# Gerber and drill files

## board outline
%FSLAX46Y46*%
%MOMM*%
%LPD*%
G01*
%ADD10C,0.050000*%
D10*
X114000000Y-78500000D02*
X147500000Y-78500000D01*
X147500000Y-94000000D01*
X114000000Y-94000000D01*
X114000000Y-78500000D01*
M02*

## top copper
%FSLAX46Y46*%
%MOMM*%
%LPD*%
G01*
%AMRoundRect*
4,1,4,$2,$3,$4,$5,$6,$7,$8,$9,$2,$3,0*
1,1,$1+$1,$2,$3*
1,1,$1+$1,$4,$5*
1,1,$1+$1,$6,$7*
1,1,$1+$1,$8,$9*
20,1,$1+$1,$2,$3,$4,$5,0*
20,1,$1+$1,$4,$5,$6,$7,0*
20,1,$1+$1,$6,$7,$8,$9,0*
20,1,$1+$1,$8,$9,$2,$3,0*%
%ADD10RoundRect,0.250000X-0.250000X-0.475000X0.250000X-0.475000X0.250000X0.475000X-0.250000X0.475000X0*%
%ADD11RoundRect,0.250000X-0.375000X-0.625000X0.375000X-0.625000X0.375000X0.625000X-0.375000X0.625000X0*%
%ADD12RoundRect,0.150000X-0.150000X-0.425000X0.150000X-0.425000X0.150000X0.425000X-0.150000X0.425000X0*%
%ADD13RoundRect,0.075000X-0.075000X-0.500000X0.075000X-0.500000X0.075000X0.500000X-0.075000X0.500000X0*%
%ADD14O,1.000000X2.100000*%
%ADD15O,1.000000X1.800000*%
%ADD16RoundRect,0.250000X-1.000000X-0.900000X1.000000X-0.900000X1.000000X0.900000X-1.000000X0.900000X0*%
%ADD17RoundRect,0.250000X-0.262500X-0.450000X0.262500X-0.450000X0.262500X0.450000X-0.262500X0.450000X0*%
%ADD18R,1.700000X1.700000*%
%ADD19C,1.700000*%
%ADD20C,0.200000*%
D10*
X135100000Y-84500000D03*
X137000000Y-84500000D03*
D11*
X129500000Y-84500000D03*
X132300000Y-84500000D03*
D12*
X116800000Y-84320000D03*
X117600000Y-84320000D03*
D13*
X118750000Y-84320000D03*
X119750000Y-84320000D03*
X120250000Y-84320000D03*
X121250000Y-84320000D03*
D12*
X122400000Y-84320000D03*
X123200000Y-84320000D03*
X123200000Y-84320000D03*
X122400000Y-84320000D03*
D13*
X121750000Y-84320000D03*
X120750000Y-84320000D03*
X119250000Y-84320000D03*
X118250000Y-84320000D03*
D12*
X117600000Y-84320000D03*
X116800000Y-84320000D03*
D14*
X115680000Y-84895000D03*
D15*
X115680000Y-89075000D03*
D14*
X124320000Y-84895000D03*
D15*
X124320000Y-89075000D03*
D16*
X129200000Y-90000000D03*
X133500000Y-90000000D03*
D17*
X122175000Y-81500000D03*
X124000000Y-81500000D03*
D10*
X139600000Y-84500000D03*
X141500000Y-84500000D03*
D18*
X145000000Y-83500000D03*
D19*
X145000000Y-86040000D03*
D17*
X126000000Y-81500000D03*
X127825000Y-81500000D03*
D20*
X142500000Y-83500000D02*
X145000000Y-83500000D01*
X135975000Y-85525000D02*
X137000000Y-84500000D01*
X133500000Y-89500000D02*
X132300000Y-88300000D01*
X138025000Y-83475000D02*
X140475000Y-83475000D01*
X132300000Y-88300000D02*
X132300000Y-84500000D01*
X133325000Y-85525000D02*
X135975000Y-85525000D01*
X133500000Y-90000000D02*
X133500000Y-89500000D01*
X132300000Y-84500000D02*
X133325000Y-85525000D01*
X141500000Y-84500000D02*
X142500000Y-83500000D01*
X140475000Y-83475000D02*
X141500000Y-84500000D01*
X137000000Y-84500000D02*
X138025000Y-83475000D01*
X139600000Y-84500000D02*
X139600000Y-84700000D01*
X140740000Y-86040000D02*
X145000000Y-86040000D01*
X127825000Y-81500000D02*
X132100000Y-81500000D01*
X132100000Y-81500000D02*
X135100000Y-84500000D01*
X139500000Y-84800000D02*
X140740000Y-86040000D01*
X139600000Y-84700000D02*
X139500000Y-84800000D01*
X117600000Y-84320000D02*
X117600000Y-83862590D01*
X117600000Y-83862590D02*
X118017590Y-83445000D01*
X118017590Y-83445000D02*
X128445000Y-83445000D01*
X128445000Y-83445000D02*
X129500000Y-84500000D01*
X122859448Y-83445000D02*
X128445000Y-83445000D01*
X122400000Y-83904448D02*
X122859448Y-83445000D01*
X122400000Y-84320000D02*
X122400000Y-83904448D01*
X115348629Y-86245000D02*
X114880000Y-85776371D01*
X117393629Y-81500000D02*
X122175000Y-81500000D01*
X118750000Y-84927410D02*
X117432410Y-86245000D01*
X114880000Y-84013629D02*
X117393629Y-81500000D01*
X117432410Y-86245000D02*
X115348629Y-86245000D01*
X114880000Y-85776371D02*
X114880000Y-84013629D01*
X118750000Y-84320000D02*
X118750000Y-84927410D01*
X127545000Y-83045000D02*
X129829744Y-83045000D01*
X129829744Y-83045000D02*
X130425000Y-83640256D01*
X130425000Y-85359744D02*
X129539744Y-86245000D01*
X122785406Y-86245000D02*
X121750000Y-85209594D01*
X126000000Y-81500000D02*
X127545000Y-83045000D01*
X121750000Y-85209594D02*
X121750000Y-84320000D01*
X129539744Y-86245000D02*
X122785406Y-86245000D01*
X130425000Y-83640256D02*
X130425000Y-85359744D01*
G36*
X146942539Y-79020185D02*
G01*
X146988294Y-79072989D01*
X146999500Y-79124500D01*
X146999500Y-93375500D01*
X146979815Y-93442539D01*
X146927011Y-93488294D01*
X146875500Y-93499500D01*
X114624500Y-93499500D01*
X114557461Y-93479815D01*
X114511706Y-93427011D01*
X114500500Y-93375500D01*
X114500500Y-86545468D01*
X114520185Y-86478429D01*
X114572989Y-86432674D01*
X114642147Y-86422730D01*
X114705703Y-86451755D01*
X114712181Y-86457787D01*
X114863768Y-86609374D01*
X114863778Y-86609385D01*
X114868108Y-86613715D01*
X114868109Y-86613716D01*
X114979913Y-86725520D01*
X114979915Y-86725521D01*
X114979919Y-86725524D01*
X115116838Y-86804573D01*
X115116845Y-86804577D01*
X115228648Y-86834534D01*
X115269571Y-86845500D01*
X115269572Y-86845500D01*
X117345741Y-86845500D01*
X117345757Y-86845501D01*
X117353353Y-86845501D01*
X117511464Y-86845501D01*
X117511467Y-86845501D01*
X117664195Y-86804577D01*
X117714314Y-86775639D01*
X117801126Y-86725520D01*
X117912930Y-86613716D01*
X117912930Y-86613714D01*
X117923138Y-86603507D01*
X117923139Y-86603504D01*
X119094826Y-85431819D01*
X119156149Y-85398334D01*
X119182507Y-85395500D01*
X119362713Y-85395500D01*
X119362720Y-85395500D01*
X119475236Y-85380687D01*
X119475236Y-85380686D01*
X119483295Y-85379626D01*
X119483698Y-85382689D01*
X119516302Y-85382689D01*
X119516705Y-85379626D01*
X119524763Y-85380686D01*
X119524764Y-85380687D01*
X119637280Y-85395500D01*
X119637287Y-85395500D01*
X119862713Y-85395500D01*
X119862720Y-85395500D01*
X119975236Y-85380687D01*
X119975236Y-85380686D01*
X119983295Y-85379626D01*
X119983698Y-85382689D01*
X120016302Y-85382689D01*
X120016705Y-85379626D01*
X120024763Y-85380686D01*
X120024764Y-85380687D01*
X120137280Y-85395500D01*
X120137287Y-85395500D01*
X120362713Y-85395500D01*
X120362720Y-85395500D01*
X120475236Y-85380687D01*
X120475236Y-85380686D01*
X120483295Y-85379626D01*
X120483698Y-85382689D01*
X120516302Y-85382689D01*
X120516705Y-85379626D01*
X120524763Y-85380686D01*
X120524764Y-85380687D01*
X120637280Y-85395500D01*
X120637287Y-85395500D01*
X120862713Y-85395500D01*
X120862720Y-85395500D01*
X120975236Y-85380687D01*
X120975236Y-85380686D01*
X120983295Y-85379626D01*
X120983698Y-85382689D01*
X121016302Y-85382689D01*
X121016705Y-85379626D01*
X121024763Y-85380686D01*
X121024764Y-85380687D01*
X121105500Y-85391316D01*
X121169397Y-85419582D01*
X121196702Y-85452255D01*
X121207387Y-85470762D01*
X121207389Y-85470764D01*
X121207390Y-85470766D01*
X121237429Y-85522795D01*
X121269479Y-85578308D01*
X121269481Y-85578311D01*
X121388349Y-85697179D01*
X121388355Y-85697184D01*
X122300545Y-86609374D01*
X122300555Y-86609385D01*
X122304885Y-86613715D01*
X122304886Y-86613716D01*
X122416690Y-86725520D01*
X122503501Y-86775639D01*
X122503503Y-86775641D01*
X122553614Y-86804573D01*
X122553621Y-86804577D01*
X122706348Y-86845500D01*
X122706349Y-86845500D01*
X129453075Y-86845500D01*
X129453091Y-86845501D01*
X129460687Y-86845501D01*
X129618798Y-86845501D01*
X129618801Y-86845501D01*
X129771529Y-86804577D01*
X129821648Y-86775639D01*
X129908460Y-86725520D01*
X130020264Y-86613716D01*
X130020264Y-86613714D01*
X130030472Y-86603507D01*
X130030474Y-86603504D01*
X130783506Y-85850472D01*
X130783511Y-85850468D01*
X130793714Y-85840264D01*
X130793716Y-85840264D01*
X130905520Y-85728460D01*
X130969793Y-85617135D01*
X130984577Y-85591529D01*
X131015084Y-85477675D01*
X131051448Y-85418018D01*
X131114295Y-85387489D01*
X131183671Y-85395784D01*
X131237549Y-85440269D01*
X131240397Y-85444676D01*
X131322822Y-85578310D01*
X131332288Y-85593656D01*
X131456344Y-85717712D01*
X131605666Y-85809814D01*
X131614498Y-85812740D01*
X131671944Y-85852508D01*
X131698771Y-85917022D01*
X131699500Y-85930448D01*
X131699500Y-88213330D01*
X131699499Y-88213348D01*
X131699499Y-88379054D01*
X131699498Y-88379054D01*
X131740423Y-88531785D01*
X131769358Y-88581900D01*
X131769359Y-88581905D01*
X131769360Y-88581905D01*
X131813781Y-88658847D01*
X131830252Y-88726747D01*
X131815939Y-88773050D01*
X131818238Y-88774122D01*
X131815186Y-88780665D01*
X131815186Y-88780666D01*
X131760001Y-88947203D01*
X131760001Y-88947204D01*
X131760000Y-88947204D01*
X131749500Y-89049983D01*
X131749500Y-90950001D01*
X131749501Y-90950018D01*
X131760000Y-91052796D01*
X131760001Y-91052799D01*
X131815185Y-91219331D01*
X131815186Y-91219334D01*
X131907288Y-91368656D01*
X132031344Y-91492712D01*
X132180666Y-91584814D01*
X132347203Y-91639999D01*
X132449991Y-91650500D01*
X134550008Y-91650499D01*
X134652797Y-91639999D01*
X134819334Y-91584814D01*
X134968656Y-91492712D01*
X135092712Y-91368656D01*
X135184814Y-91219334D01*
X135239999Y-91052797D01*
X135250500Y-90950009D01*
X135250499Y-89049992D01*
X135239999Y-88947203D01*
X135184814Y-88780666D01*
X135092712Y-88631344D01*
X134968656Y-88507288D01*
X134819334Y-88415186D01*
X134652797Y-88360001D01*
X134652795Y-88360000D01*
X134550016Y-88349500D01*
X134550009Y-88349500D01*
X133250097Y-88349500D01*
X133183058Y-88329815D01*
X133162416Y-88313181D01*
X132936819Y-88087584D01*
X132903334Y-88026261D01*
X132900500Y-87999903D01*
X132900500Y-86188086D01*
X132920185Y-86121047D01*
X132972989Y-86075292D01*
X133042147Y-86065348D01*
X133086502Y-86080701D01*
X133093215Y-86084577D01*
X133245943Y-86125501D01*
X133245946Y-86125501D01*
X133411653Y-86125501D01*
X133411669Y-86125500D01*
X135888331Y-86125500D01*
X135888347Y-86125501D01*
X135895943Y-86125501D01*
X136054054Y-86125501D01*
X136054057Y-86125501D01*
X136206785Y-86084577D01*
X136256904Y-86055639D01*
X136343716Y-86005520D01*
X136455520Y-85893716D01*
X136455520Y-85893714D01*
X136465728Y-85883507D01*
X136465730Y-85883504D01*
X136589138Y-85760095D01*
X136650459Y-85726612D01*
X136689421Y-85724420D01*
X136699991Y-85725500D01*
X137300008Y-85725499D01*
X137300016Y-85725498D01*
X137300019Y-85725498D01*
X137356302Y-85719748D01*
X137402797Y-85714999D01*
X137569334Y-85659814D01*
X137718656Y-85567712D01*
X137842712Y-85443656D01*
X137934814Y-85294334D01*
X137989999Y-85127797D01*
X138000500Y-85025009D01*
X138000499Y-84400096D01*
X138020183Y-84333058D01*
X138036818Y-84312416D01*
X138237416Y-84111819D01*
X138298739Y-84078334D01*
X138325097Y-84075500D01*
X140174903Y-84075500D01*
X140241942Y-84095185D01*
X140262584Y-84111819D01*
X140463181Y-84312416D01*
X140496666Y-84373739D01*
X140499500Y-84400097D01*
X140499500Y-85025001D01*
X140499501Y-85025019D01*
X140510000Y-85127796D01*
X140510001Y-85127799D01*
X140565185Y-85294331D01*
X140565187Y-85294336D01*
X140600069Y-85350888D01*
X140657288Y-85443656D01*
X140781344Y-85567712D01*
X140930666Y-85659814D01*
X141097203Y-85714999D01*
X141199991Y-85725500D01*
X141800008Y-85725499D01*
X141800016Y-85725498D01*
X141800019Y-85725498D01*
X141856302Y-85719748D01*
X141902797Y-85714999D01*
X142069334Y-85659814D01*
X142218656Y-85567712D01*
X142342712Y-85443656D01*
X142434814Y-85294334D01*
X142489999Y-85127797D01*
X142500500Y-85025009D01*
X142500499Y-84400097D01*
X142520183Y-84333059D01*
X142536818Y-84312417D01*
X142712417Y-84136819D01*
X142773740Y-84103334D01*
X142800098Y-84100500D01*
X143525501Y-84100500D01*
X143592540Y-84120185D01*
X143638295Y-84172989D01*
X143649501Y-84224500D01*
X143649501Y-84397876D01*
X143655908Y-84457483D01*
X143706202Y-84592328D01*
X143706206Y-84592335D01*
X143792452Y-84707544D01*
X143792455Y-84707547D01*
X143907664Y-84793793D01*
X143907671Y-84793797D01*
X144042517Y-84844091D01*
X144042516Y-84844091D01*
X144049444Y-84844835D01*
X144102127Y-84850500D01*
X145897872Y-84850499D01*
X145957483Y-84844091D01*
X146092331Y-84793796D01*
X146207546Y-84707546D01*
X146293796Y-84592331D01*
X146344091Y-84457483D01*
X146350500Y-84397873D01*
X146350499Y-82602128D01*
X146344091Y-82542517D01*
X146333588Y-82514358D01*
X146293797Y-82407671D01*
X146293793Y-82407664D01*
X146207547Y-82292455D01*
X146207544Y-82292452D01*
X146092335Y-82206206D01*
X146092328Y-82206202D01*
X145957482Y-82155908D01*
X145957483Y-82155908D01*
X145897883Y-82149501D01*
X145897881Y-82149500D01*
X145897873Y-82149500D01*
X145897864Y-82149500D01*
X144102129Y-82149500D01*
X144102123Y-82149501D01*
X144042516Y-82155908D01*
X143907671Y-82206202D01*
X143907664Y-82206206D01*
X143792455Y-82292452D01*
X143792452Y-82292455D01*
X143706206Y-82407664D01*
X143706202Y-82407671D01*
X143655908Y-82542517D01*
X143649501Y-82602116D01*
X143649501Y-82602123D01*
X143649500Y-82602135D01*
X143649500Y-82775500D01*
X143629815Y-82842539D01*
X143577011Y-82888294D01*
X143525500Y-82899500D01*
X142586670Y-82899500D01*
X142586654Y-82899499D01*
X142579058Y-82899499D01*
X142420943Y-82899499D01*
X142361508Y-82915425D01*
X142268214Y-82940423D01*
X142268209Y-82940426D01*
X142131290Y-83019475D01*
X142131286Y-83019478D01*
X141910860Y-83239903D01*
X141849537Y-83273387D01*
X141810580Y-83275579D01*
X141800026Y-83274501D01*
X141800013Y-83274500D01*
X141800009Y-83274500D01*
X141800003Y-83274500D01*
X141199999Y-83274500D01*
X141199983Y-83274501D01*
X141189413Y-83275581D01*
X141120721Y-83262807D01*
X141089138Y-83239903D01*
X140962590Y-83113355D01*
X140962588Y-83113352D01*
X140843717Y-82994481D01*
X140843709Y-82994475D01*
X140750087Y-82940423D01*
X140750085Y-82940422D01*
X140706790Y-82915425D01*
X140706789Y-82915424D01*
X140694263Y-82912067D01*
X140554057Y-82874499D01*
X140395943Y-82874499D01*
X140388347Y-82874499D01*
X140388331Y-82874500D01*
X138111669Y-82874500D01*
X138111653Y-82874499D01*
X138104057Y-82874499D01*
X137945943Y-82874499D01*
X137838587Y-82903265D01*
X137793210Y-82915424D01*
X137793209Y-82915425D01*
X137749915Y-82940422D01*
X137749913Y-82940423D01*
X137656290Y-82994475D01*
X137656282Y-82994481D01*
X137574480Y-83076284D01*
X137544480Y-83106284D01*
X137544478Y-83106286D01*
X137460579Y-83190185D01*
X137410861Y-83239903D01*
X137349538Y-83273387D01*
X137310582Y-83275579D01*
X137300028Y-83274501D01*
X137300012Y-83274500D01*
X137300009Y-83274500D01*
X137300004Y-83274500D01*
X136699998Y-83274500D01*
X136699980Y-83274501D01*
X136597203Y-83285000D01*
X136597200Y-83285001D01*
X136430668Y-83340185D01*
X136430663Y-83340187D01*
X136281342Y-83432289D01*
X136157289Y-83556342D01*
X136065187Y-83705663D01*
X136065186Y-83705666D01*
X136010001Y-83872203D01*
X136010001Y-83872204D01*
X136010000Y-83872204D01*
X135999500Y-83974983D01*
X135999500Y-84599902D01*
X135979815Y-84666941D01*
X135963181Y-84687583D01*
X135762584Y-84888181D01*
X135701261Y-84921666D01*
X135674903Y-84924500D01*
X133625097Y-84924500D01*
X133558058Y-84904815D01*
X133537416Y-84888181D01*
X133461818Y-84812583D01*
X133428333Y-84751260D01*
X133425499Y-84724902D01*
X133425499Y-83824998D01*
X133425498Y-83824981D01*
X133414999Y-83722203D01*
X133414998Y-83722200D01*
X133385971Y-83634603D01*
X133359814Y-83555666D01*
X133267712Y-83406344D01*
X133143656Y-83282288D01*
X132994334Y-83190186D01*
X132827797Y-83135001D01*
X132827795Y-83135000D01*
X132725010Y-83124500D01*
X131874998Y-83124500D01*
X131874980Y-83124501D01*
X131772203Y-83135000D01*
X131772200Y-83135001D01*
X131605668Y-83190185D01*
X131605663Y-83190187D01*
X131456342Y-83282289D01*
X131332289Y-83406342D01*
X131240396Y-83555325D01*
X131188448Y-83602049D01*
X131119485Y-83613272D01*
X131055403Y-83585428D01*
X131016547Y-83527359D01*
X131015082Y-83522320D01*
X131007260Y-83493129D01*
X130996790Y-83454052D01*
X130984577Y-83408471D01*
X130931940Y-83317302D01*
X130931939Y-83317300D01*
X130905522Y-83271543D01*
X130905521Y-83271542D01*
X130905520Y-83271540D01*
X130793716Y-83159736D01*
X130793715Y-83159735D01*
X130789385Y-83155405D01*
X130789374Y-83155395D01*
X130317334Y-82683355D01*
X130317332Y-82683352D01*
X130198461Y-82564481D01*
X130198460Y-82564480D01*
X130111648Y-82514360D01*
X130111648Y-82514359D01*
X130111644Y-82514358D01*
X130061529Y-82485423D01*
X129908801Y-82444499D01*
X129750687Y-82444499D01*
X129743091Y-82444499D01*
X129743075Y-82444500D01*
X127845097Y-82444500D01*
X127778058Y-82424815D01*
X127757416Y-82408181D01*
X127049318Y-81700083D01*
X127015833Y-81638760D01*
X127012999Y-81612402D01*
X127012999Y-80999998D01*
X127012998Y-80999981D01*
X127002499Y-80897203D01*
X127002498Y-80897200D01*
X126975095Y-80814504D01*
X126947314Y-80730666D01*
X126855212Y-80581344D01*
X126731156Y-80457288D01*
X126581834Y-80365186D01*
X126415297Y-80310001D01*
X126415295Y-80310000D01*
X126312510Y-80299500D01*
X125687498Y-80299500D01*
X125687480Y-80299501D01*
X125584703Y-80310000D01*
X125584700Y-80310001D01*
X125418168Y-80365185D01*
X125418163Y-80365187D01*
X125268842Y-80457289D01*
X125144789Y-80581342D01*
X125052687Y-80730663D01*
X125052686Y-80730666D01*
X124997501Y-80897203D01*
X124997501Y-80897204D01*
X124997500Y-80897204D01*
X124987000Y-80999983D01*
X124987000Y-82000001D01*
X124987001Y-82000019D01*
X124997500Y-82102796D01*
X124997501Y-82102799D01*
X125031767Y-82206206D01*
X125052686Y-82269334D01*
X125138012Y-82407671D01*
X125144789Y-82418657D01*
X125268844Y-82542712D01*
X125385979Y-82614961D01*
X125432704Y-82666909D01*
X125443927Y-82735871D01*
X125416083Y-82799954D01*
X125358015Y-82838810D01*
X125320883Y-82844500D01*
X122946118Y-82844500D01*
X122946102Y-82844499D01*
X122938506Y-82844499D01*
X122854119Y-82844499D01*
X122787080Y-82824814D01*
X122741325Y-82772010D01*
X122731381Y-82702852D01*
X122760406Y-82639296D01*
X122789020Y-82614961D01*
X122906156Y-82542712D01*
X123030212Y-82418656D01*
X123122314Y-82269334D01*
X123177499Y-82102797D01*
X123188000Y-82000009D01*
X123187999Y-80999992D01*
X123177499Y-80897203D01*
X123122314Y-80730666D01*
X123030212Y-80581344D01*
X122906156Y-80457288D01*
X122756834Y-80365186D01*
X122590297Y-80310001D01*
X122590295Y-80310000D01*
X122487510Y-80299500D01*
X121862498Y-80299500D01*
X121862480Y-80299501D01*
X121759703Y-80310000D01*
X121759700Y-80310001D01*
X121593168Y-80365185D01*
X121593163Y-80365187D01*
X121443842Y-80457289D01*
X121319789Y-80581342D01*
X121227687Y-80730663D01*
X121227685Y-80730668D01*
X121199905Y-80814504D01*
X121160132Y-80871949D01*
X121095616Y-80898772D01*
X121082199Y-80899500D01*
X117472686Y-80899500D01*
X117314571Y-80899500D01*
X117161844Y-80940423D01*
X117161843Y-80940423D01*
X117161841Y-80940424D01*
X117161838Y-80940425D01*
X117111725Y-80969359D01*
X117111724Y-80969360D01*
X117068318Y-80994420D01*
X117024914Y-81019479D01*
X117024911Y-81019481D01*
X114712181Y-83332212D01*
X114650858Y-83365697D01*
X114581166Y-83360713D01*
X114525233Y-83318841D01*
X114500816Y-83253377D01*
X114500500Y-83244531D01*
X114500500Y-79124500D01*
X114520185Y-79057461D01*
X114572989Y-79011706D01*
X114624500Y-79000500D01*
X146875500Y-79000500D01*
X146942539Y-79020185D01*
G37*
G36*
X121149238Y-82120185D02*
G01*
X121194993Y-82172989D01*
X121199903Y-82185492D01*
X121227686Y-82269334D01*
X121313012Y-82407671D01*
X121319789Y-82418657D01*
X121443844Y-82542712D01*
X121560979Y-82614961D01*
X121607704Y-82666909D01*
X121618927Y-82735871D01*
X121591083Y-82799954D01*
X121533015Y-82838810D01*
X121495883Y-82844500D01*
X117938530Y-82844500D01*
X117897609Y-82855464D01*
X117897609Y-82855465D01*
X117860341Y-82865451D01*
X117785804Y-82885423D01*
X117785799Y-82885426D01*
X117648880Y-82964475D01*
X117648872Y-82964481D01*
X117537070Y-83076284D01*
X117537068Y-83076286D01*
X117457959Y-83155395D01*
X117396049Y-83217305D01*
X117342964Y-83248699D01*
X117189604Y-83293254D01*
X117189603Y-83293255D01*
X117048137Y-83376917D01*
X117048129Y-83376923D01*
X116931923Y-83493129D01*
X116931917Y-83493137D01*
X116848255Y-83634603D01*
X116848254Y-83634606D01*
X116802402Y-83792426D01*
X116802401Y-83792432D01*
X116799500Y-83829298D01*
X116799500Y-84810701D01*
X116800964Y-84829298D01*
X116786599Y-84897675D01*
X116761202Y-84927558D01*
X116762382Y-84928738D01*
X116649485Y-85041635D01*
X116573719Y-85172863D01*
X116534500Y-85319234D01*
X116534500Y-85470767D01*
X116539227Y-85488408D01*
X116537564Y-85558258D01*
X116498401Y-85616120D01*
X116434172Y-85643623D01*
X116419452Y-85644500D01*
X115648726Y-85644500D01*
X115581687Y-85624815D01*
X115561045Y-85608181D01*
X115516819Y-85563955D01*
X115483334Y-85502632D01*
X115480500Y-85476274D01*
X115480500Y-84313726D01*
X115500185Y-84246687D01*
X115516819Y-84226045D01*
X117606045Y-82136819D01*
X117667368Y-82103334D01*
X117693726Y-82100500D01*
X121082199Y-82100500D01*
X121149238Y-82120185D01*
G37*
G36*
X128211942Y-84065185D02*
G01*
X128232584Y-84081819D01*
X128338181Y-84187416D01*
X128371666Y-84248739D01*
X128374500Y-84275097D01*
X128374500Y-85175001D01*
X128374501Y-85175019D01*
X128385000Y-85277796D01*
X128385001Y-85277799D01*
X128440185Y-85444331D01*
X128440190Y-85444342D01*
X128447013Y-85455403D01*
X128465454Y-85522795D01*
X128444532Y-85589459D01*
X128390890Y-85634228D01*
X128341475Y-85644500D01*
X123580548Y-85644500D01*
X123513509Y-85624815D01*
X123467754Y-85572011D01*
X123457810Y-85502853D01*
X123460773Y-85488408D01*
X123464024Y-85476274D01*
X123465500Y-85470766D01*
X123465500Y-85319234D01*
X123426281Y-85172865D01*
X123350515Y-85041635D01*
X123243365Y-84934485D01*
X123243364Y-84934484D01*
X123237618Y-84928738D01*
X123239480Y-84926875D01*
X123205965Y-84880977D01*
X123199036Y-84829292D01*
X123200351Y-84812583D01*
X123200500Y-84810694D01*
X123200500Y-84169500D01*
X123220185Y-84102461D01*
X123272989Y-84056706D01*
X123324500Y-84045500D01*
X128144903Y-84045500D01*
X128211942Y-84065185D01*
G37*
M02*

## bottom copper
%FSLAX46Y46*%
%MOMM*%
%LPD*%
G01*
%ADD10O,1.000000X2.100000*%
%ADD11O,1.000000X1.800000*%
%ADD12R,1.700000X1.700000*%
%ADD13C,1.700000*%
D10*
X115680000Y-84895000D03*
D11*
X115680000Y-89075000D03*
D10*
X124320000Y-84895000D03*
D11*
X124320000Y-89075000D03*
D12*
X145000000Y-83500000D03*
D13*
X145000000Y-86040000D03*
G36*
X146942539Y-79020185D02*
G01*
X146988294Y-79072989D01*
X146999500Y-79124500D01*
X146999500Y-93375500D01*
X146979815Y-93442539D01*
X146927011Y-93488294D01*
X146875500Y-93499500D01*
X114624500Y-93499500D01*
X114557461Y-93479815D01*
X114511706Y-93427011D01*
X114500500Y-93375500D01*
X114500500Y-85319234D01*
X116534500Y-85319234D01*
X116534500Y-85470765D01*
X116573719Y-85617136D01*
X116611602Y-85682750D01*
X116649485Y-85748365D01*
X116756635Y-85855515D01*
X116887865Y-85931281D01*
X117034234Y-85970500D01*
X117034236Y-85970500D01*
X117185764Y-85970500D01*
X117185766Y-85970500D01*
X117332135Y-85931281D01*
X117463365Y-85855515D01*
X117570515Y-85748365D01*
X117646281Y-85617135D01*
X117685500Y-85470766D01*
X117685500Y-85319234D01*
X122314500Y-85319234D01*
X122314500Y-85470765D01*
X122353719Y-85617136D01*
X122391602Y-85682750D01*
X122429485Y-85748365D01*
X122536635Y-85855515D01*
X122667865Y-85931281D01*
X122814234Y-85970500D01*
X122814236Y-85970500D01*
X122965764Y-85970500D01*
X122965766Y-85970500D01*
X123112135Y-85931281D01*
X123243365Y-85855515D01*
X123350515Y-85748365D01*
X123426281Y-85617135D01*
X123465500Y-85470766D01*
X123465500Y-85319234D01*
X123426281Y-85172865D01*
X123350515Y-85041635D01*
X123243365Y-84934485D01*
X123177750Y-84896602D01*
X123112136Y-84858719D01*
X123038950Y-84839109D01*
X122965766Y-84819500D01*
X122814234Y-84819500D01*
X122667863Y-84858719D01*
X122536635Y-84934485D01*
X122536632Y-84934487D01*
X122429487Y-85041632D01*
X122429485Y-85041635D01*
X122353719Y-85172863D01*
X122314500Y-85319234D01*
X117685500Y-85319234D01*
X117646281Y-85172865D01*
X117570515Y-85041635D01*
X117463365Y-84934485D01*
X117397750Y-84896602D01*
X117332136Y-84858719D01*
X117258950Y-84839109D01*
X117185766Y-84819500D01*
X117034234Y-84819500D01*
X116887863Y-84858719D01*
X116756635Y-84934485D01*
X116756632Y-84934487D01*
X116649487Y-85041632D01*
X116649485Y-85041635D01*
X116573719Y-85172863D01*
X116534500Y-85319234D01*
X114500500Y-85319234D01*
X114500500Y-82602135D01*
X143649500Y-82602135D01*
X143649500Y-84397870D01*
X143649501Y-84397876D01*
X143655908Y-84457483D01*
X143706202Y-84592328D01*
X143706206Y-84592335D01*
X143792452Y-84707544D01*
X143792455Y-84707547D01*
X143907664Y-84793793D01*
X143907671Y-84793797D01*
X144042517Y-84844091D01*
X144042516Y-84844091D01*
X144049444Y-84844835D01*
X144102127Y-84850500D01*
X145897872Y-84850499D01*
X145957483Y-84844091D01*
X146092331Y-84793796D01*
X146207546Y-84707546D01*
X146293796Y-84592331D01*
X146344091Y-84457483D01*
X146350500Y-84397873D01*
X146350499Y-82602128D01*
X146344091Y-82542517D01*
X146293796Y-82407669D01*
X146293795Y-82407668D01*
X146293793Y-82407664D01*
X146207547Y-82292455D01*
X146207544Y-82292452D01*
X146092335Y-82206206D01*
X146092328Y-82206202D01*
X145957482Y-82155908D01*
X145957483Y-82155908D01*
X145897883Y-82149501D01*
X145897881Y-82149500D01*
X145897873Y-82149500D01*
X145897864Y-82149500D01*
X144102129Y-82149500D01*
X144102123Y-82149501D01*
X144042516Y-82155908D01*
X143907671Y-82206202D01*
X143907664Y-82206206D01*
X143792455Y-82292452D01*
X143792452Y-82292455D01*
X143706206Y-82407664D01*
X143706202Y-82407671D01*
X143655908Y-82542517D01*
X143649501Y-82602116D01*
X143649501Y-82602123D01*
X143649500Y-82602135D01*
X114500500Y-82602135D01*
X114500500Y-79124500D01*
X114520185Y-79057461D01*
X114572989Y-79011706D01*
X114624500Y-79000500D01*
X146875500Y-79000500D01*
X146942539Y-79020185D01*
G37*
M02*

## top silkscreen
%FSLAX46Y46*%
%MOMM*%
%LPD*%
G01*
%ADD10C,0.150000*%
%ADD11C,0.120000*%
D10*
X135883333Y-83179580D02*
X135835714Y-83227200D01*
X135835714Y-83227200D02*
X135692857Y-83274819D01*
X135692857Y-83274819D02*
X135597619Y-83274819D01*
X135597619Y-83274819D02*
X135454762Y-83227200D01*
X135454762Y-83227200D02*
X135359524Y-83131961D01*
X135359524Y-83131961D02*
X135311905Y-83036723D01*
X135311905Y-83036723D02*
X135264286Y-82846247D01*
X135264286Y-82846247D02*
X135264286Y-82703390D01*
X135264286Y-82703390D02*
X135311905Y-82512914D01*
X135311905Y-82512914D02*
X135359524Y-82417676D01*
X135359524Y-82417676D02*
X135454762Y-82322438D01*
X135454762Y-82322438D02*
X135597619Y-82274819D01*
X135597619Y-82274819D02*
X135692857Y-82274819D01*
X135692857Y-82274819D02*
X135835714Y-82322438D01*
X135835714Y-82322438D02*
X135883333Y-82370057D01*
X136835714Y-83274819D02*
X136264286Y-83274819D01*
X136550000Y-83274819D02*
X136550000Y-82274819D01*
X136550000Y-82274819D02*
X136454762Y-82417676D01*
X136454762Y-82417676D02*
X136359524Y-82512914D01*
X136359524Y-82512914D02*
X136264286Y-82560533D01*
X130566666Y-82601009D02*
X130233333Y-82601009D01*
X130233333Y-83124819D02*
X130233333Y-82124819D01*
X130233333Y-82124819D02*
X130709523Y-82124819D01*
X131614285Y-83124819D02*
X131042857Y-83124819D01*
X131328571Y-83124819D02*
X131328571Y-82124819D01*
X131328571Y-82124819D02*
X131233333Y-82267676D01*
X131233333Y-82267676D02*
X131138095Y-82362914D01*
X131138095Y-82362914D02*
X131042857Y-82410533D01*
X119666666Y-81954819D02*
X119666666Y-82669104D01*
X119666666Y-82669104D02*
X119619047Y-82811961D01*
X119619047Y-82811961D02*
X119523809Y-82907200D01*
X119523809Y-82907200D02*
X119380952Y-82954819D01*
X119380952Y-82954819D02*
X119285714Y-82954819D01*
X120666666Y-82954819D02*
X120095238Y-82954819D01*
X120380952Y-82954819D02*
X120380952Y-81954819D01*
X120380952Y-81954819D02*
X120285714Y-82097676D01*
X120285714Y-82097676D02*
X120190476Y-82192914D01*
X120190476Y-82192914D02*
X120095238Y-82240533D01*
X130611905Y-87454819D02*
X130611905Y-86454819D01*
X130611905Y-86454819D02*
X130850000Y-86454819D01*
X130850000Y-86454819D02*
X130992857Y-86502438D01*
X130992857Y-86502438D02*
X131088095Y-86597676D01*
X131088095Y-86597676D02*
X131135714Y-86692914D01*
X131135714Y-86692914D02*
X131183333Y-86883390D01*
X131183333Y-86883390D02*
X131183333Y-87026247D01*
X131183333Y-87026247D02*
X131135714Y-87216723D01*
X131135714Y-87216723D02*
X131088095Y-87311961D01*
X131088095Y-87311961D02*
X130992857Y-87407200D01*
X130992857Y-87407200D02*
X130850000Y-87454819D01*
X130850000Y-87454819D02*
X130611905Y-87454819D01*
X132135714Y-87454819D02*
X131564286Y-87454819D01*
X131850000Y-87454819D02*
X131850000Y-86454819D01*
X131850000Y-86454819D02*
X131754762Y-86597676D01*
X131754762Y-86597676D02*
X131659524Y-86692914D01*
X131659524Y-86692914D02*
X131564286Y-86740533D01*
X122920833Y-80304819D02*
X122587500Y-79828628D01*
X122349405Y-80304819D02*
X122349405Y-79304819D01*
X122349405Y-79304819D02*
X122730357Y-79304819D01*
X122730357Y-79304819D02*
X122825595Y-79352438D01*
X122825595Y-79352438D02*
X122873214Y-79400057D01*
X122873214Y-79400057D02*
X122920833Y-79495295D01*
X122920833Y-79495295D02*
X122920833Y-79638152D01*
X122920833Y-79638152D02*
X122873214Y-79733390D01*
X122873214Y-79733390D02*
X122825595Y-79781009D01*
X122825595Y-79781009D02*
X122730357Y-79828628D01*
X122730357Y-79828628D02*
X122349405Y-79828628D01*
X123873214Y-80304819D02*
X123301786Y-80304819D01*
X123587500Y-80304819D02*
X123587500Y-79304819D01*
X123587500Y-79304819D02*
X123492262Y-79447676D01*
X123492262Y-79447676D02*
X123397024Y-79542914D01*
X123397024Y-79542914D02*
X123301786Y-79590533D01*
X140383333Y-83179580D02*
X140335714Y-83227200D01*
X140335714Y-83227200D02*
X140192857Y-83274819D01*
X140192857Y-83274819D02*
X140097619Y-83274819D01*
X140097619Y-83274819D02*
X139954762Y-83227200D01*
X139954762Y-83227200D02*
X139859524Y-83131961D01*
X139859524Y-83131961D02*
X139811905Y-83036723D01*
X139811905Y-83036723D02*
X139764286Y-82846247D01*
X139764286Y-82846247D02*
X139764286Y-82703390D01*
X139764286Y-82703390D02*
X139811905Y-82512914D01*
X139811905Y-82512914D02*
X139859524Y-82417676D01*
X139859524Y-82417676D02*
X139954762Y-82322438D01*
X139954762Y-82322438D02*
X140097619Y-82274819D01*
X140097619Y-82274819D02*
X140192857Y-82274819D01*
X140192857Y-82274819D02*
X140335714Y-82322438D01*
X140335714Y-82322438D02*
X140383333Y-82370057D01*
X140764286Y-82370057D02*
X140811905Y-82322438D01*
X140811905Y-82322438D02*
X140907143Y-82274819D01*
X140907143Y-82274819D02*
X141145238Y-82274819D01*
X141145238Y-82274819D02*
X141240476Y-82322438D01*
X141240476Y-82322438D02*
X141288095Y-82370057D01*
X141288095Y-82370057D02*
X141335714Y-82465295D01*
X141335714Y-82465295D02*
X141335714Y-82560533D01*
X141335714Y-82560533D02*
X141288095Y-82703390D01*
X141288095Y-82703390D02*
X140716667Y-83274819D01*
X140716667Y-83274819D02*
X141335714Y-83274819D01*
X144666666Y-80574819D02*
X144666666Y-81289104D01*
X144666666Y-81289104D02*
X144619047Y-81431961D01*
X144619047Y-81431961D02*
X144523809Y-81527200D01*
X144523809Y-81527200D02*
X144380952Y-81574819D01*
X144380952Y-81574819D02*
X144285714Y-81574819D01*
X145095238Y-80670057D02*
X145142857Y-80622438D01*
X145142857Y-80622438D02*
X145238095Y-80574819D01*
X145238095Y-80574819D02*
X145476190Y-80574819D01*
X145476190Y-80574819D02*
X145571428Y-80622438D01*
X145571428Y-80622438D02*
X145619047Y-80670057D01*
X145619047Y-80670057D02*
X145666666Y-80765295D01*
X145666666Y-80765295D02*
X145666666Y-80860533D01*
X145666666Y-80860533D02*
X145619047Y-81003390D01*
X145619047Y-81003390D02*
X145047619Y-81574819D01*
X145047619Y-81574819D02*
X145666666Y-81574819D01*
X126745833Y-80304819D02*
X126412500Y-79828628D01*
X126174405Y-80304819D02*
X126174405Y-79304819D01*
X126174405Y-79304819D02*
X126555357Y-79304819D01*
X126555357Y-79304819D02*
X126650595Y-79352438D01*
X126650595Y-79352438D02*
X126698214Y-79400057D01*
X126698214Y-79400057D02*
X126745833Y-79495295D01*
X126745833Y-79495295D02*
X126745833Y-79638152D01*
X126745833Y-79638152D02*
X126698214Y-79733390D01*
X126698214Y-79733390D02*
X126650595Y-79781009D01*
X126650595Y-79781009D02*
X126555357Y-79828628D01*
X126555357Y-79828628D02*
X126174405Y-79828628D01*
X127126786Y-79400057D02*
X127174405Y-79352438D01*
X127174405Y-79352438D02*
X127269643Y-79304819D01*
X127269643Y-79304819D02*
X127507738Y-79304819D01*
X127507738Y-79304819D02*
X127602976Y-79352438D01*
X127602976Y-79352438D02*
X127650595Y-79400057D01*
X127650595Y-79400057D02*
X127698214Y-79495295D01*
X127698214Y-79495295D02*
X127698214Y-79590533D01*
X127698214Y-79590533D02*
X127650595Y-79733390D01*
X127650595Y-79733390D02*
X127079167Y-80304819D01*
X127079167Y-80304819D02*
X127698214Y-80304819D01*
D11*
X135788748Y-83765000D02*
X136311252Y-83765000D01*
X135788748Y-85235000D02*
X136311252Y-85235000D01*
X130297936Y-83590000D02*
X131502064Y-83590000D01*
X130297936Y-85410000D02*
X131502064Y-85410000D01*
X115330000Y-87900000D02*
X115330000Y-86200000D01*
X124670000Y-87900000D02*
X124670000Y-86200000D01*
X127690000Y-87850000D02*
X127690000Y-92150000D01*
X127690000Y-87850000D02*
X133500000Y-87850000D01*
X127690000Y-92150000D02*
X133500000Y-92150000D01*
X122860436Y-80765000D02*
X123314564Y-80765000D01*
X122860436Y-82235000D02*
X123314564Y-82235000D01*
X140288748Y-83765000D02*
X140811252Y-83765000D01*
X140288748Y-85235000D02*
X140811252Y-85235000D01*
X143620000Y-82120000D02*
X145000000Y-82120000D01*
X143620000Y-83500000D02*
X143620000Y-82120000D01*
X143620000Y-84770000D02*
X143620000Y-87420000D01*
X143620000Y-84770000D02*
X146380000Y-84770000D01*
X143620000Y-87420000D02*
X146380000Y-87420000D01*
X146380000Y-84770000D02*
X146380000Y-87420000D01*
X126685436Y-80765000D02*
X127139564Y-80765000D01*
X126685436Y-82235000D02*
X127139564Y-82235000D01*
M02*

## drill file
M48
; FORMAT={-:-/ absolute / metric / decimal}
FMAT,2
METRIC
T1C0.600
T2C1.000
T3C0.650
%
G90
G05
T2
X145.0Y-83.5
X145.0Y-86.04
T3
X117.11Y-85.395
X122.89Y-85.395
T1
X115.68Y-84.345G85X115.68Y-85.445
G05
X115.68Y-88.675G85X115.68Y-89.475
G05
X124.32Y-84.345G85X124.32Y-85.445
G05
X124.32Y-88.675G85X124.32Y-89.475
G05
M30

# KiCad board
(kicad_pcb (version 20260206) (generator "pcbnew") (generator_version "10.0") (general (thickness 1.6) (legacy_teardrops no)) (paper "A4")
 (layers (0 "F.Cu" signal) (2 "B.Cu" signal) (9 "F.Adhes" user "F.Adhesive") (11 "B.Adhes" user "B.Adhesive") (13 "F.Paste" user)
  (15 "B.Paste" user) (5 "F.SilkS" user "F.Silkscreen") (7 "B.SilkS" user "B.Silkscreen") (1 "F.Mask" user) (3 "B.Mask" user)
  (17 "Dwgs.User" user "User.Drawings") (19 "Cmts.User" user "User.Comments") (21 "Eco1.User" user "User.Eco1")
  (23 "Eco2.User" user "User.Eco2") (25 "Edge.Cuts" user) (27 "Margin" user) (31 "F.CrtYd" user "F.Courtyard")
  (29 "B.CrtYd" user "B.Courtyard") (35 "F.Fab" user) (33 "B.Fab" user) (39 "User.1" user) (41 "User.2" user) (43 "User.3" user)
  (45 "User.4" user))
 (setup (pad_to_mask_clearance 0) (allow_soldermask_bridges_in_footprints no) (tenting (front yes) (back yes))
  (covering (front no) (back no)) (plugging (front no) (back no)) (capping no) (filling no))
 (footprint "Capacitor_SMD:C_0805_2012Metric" (layer "F.Cu") (at 136.05 84.5)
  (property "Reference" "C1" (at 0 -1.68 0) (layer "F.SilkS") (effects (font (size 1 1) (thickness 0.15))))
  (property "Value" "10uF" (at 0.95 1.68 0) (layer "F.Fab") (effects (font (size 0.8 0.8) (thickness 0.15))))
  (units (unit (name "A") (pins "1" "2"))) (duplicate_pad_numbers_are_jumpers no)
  (fp_line (start -0.261252 -0.735) (end 0.261252 -0.735) (stroke (width 0.12) (type solid)) (layer "F.SilkS"))
  (fp_line (start -0.261252 0.735) (end 0.261252 0.735) (stroke (width 0.12) (type solid)) (layer "F.SilkS"))
  (pad "1" smd roundrect (at -0.95 0) (size 1 1.45) (layers "F.Cu" "F.Mask" "F.Paste") (roundrect_rratio 0.25) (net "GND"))
  (pad "2" smd roundrect (at 0.95 0) (size 1 1.45) (layers "F.Cu" "F.Mask" "F.Paste") (roundrect_rratio 0.25) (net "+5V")))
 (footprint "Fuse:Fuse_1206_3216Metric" (layer "F.Cu") (at 130.9 84.5)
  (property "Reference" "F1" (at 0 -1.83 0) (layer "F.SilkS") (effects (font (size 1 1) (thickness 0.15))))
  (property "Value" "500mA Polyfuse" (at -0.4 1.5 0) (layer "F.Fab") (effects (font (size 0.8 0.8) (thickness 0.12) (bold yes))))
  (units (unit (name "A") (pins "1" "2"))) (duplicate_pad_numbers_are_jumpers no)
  (fp_line (start -0.602064 -0.91) (end 0.602064 -0.91) (stroke (width 0.12) (type solid)) (layer "F.SilkS"))
  (fp_line (start -0.602064 0.91) (end 0.602064 0.91) (stroke (width 0.12) (type solid)) (layer "F.SilkS"))
  (pad "1" smd roundrect (at -1.4 0) (size 1.25 1.75) (layers "F.Cu" "F.Mask" "F.Paste") (roundrect_rratio 0.2) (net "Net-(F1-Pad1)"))
  (pad "2" smd roundrect (at 1.4 0) (size 1.25 1.75) (layers "F.Cu" "F.Mask" "F.Paste") (roundrect_rratio 0.2) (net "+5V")))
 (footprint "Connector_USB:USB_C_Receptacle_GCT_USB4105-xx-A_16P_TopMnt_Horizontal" (layer "F.Cu") (at 120 88)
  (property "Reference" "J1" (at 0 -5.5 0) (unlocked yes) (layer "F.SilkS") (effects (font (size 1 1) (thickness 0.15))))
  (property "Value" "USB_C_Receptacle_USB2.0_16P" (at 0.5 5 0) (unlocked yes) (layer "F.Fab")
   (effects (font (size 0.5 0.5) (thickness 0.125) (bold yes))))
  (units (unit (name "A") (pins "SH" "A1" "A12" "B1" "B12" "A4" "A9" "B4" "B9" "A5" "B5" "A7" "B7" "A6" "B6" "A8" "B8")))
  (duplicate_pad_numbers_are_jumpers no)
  (fp_line (start -4.67 -0.1) (end -4.67 -1.8) (stroke (width 0.12) (type solid)) (layer "F.SilkS"))
  (fp_line (start 4.67 -0.1) (end 4.67 -1.8) (stroke (width 0.12) (type solid)) (layer "F.SilkS"))
  (pad "" np_thru_hole circle (at -2.89 -2.605) (size 0.65 0.65) (drill 0.65) (layers "*.Cu" "*.Mask"))
  (pad "" np_thru_hole circle (at 2.89 -2.605) (size 0.65 0.65) (drill 0.65) (layers "*.Cu" "*.Mask"))
  (pad "A1" smd roundrect (at -3.2 -3.68) (size 0.6 1.15) (layers "F.Cu" "F.Mask" "F.Paste") (roundrect_rratio 0.25) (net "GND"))
  (pad "A4" smd roundrect (at -2.4 -3.68) (size 0.6 1.15) (layers "F.Cu" "F.Mask" "F.Paste") (roundrect_rratio 0.25) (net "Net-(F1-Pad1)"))
  (pad "A5" smd roundrect (at -1.25 -3.68) (size 0.3 1.15) (layers "F.Cu" "F.Mask" "F.Paste") (roundrect_rratio 0.25) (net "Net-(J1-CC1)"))
  (pad "A6" smd roundrect (at -0.25 -3.68) (size 0.3 1.15) (layers "F.Cu" "F.Mask" "F.Paste") (roundrect_rratio 0.25)
   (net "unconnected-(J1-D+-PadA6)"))
  (pad "A7" smd roundrect (at 0.25 -3.68) (size 0.3 1.15) (layers "F.Cu" "F.Mask" "F.Paste") (roundrect_rratio 0.25)
   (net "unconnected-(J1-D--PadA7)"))
  (pad "A8" smd roundrect (at 1.25 -3.68) (size 0.3 1.15) (layers "F.Cu" "F.Mask" "F.Paste") (roundrect_rratio 0.25)
   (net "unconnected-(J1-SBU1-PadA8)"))
  (pad "A9" smd roundrect (at 2.4 -3.68) (size 0.6 1.15) (layers "F.Cu" "F.Mask" "F.Paste") (roundrect_rratio 0.25) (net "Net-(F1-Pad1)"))
  (pad "A12" smd roundrect (at 3.2 -3.68) (size 0.6 1.15) (layers "F.Cu" "F.Mask" "F.Paste") (roundrect_rratio 0.25) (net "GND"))
  (pad "B1" smd roundrect (at 3.2 -3.68) (size 0.6 1.15) (layers "F.Cu" "F.Mask" "F.Paste") (roundrect_rratio 0.25) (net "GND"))
  (pad "B4" smd roundrect (at 2.4 -3.68) (size 0.6 1.15) (layers "F.Cu" "F.Mask" "F.Paste") (roundrect_rratio 0.25) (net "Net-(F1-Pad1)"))
  (pad "B5" smd roundrect (at 1.75 -3.68) (size 0.3 1.15) (layers "F.Cu" "F.Mask" "F.Paste") (roundrect_rratio 0.25) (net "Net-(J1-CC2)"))
  (pad "B6" smd roundrect (at 0.75 -3.68) (size 0.3 1.15) (layers "F.Cu" "F.Mask" "F.Paste") (roundrect_rratio 0.25)
   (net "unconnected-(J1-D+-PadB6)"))
  (pad "B7" smd roundrect (at -0.75 -3.68) (size 0.3 1.15) (layers "F.Cu" "F.Mask" "F.Paste") (roundrect_rratio 0.25)
   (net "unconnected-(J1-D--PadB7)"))
  (pad "B8" smd roundrect (at -1.75 -3.68) (size 0.3 1.15) (layers "F.Cu" "F.Mask" "F.Paste") (roundrect_rratio 0.25)
   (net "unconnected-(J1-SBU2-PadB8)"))
  (pad "B9" smd roundrect (at -2.4 -3.68) (size 0.6 1.15) (layers "F.Cu" "F.Mask" "F.Paste") (roundrect_rratio 0.25) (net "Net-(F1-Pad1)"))
  (pad "B12" smd roundrect (at -3.2 -3.68) (size 0.6 1.15) (layers "F.Cu" "F.Mask" "F.Paste") (roundrect_rratio 0.25) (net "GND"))
  (pad "SH" thru_hole oval (at -4.32 -3.105) (size 1 2.1) (drill oval 0.6 1.7) (layers "*.Cu" "*.Mask" "F.Paste") (remove_unused_layers no)
   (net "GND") (zone_connect 2))
  (pad "SH" thru_hole oval (at -4.32 1.075) (size 1 1.8) (drill oval 0.6 1.4) (layers "*.Cu" "*.Mask" "F.Paste") (remove_unused_layers no)
   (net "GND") (zone_connect 2))
  (pad "SH" thru_hole oval (at 4.32 -3.105) (size 1 2.1) (drill oval 0.6 1.7) (layers "*.Cu" "*.Mask" "F.Paste") (remove_unused_layers no)
   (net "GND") (zone_connect 2))
  (pad "SH" thru_hole oval (at 4.32 1.075) (size 1 1.8) (drill oval 0.6 1.4) (layers "*.Cu" "*.Mask" "F.Paste") (remove_unused_layers no)
   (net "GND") (zone_connect 2)))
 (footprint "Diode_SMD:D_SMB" (layer "F.Cu") (at 131.35 90)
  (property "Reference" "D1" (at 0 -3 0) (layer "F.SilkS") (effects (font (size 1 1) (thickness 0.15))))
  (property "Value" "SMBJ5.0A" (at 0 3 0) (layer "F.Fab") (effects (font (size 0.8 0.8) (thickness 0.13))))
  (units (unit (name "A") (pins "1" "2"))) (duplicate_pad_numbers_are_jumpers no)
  (fp_line (start -3.66 -2.15) (end -3.66 2.15) (stroke (width 0.12) (type solid)) (layer "F.SilkS"))
  (fp_line (start -3.66 -2.15) (end 2.15 -2.15) (stroke (width 0.12) (type solid)) (layer "F.SilkS"))
  (fp_line (start -3.66 2.15) (end 2.15 2.15) (stroke (width 0.12) (type solid)) (layer "F.SilkS"))
  (pad "1" smd roundrect (at -2.15 0) (size 2.5 2.3) (layers "F.Cu" "F.Mask" "F.Paste") (roundrect_rratio 0.1086956522) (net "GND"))
  (pad "2" smd roundrect (at 2.15 0) (size 2.5 2.3) (layers "F.Cu" "F.Mask" "F.Paste") (roundrect_rratio 0.1086956522) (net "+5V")))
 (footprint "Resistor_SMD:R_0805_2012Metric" (layer "F.Cu") (at 123.0875 81.5)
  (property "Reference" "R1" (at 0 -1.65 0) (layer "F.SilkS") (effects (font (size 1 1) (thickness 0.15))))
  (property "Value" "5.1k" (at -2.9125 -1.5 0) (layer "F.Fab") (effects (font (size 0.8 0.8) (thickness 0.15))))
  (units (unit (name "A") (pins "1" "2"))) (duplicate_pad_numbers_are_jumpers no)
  (fp_line (start -0.227064 -0.735) (end 0.227064 -0.735) (stroke (width 0.12) (type solid)) (layer "F.SilkS"))
  (fp_line (start -0.227064 0.735) (end 0.227064 0.735) (stroke (width 0.12) (type solid)) (layer "F.SilkS"))
  (pad "1" smd roundrect (at -0.9125 0) (size 1.025 1.4) (layers "F.Cu" "F.Mask" "F.Paste") (roundrect_rratio 0.243902) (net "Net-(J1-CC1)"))
  (pad "2" smd roundrect (at 0.9125 0) (size 1.025 1.4) (layers "F.Cu" "F.Mask" "F.Paste") (roundrect_rratio 0.243902) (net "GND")))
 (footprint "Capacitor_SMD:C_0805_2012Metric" (layer "F.Cu") (at 140.55 84.5)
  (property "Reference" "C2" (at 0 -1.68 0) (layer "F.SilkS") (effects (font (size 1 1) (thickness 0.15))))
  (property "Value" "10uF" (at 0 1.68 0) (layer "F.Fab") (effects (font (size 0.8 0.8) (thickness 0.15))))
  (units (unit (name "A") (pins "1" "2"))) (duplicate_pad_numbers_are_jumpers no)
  (fp_line (start -0.261252 -0.735) (end 0.261252 -0.735) (stroke (width 0.12) (type solid)) (layer "F.SilkS"))
  (fp_line (start -0.261252 0.735) (end 0.261252 0.735) (stroke (width 0.12) (type solid)) (layer "F.SilkS"))
  (pad "1" smd roundrect (at -0.95 0) (size 1 1.45) (layers "F.Cu" "F.Mask" "F.Paste") (roundrect_rratio 0.25) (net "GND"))
  (pad "2" smd roundrect (at 0.95 0) (size 1 1.45) (layers "F.Cu" "F.Mask" "F.Paste") (roundrect_rratio 0.25) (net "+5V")))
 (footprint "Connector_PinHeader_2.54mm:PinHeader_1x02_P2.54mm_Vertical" (layer "F.Cu") (at 145 83.5)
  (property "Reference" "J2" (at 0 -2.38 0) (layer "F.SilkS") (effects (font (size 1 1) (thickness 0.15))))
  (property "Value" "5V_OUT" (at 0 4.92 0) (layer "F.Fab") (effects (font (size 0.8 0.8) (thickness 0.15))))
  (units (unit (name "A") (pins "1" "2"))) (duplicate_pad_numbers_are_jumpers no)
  (fp_line (start -1.38 -1.38) (end 0 -1.38) (stroke (width 0.12) (type solid)) (layer "F.SilkS"))
  (fp_line (start -1.38 0) (end -1.38 -1.38) (stroke (width 0.12) (type solid)) (layer "F.SilkS"))
  (fp_line (start -1.38 1.27) (end -1.38 3.92) (stroke (width 0.12) (type solid)) (layer "F.SilkS"))
  (fp_line (start -1.38 1.27) (end 1.38 1.27) (stroke (width 0.12) (type solid)) (layer "F.SilkS"))
  (fp_line (start -1.38 3.92) (end 1.38 3.92) (stroke (width 0.12) (type solid)) (layer "F.SilkS"))
  (fp_line (start 1.38 1.27) (end 1.38 3.92) (stroke (width 0.12) (type solid)) (layer "F.SilkS"))
  (pad "1" thru_hole rect (at 0 0) (size 1.7 1.7) (drill 1) (layers "*.Cu" "*.Mask") (remove_unused_layers no) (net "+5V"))
  (pad "2" thru_hole circle (at 0 2.54) (size 1.7 1.7) (drill 1) (layers "*.Cu" "*.Mask") (remove_unused_layers no) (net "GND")))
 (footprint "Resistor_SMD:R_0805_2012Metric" (layer "F.Cu") (at 126.9125 81.5)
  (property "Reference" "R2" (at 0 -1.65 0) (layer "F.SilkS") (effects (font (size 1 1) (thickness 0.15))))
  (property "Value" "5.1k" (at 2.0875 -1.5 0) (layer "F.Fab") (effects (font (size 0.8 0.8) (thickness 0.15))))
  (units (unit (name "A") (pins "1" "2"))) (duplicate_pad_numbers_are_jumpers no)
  (fp_line (start -0.227064 -0.735) (end 0.227064 -0.735) (stroke (width 0.12) (type solid)) (layer "F.SilkS"))
  (fp_line (start -0.227064 0.735) (end 0.227064 0.735) (stroke (width 0.12) (type solid)) (layer "F.SilkS"))
  (pad "1" smd roundrect (at -0.9125 0) (size 1.025 1.4) (layers "F.Cu" "F.Mask" "F.Paste") (roundrect_rratio 0.243902) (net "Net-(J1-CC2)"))
  (pad "2" smd roundrect (at 0.9125 0) (size 1.025 1.4) (layers "F.Cu" "F.Mask" "F.Paste") (roundrect_rratio 0.243902) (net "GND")))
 (gr_rect (start 114 78.5) (end 147.5 94) (stroke (width 0.05) (type default)) (fill no) (layer "Edge.Cuts"))
 (segment (start 142.5 83.5) (end 145 83.5) (width 0.2) (layer "F.Cu") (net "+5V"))
 (segment (start 135.975 85.525) (end 137 84.5) (width 0.2) (layer "F.Cu") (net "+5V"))
 (segment (start 133.5 89.5) (end 132.3 88.3) (width 0.2) (layer "F.Cu") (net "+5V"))
 (segment (start 138.025 83.475) (end 140.475 83.475) (width 0.2) (layer "F.Cu") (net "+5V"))
 (segment (start 132.3 88.3) (end 132.3 84.5) (width 0.2) (layer "F.Cu") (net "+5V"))
 (segment (start 133.325 85.525) (end 135.975 85.525) (width 0.2) (layer "F.Cu") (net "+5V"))
 (segment (start 133.5 90) (end 133.5 89.5) (width 0.2) (layer "F.Cu") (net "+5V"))
 (segment (start 132.3 84.5) (end 133.325 85.525) (width 0.2) (layer "F.Cu") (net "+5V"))
 (segment (start 141.5 84.5) (end 142.5 83.5) (width 0.2) (layer "F.Cu") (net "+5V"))
 (segment (start 140.475 83.475) (end 141.5 84.5) (width 0.2) (layer "F.Cu") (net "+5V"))
 (segment (start 137 84.5) (end 138.025 83.475) (width 0.2) (layer "F.Cu") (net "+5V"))
 (segment (start 139.6 84.5) (end 139.6 84.7) (width 0.2) (layer "F.Cu") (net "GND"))
 (segment (start 140.74 86.04) (end 145 86.04) (width 0.2) (layer "F.Cu") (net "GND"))
 (segment (start 127.825 81.5) (end 132.1 81.5) (width 0.2) (layer "F.Cu") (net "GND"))
 (segment (start 132.1 81.5) (end 135.1 84.5) (width 0.2) (layer "F.Cu") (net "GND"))
 (segment (start 139.5 84.8) (end 140.74 86.04) (width 0.2) (layer "F.Cu") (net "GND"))
 (segment (start 139.6 84.7) (end 139.5 84.8) (width 0.2) (layer "F.Cu") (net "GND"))
 (segment (start 117.6 84.32) (end 117.6 83.86259) (width 0.2) (layer "F.Cu") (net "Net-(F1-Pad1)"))
 (segment (start 117.6 83.86259) (end 118.01759 83.445) (width 0.2) (layer "F.Cu") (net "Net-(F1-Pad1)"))
 (segment (start 118.01759 83.445) (end 128.445 83.445) (width 0.2) (layer "F.Cu") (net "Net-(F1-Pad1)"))
 (segment (start 128.445 83.445) (end 129.5 84.5) (width 0.2) (layer "F.Cu") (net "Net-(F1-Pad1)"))
 (segment (start 122.859448 83.445) (end 128.445 83.445) (width 0.2) (layer "F.Cu") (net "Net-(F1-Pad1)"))
 (segment (start 122.4 83.904448) (end 122.859448 83.445) (width 0.2) (layer "F.Cu") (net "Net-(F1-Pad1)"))
 (segment (start 122.4 84.32) (end 122.4 83.904448) (width 0.2) (layer "F.Cu") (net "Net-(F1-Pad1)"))
 (segment (start 115.348629 86.245) (end 114.88 85.776371) (width 0.2) (layer "F.Cu") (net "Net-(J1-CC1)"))
 (segment (start 117.393629 81.5) (end 122.175 81.5) (width 0.2) (layer "F.Cu") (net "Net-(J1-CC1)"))
 (segment (start 118.75 84.92741) (end 117.43241 86.245) (width 0.2) (layer "F.Cu") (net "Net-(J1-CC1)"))
 (segment (start 114.88 84.013629) (end 117.393629 81.5) (width 0.2) (layer "F.Cu") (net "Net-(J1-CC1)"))
 (segment (start 117.43241 86.245) (end 115.348629 86.245) (width 0.2) (layer "F.Cu") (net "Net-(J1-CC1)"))
 (segment (start 114.88 85.776371) (end 114.88 84.013629) (width 0.2) (layer "F.Cu") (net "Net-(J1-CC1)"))
 (segment (start 118.75 84.32) (end 118.75 84.92741) (width 0.2) (layer "F.Cu") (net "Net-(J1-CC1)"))
 (segment (start 127.545 83.045) (end 129.829744 83.045) (width 0.2) (layer "F.Cu") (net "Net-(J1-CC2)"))
 (segment (start 129.829744 83.045) (end 130.425 83.640256) (width 0.2) (layer "F.Cu") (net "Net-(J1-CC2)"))
 (segment (start 130.425 85.359744) (end 129.539744 86.245) (width 0.2) (layer "F.Cu") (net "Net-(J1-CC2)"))
 (segment (start 122.785406 86.245) (end 121.75 85.209594) (width 0.2) (layer "F.Cu") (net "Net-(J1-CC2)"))
 (segment (start 126 81.5) (end 127.545 83.045) (width 0.2) (layer "F.Cu") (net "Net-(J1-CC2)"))
 (segment (start 121.75 85.209594) (end 121.75 84.32) (width 0.2) (layer "F.Cu") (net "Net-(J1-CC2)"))
 (segment (start 129.539744 86.245) (end 122.785406 86.245) (width 0.2) (layer "F.Cu") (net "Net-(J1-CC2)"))
 (segment (start 130.425 83.640256) (end 130.425 85.359744) (width 0.2) (layer "F.Cu") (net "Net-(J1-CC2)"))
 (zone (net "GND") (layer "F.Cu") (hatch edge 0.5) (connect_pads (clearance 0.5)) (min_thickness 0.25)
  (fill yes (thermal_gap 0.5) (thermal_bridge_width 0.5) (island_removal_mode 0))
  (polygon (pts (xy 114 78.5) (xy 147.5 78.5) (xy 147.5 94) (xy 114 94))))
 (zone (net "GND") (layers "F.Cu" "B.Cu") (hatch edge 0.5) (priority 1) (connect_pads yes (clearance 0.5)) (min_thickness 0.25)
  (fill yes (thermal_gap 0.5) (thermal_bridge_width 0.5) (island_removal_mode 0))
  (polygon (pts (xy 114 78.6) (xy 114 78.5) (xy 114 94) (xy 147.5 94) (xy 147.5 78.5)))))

